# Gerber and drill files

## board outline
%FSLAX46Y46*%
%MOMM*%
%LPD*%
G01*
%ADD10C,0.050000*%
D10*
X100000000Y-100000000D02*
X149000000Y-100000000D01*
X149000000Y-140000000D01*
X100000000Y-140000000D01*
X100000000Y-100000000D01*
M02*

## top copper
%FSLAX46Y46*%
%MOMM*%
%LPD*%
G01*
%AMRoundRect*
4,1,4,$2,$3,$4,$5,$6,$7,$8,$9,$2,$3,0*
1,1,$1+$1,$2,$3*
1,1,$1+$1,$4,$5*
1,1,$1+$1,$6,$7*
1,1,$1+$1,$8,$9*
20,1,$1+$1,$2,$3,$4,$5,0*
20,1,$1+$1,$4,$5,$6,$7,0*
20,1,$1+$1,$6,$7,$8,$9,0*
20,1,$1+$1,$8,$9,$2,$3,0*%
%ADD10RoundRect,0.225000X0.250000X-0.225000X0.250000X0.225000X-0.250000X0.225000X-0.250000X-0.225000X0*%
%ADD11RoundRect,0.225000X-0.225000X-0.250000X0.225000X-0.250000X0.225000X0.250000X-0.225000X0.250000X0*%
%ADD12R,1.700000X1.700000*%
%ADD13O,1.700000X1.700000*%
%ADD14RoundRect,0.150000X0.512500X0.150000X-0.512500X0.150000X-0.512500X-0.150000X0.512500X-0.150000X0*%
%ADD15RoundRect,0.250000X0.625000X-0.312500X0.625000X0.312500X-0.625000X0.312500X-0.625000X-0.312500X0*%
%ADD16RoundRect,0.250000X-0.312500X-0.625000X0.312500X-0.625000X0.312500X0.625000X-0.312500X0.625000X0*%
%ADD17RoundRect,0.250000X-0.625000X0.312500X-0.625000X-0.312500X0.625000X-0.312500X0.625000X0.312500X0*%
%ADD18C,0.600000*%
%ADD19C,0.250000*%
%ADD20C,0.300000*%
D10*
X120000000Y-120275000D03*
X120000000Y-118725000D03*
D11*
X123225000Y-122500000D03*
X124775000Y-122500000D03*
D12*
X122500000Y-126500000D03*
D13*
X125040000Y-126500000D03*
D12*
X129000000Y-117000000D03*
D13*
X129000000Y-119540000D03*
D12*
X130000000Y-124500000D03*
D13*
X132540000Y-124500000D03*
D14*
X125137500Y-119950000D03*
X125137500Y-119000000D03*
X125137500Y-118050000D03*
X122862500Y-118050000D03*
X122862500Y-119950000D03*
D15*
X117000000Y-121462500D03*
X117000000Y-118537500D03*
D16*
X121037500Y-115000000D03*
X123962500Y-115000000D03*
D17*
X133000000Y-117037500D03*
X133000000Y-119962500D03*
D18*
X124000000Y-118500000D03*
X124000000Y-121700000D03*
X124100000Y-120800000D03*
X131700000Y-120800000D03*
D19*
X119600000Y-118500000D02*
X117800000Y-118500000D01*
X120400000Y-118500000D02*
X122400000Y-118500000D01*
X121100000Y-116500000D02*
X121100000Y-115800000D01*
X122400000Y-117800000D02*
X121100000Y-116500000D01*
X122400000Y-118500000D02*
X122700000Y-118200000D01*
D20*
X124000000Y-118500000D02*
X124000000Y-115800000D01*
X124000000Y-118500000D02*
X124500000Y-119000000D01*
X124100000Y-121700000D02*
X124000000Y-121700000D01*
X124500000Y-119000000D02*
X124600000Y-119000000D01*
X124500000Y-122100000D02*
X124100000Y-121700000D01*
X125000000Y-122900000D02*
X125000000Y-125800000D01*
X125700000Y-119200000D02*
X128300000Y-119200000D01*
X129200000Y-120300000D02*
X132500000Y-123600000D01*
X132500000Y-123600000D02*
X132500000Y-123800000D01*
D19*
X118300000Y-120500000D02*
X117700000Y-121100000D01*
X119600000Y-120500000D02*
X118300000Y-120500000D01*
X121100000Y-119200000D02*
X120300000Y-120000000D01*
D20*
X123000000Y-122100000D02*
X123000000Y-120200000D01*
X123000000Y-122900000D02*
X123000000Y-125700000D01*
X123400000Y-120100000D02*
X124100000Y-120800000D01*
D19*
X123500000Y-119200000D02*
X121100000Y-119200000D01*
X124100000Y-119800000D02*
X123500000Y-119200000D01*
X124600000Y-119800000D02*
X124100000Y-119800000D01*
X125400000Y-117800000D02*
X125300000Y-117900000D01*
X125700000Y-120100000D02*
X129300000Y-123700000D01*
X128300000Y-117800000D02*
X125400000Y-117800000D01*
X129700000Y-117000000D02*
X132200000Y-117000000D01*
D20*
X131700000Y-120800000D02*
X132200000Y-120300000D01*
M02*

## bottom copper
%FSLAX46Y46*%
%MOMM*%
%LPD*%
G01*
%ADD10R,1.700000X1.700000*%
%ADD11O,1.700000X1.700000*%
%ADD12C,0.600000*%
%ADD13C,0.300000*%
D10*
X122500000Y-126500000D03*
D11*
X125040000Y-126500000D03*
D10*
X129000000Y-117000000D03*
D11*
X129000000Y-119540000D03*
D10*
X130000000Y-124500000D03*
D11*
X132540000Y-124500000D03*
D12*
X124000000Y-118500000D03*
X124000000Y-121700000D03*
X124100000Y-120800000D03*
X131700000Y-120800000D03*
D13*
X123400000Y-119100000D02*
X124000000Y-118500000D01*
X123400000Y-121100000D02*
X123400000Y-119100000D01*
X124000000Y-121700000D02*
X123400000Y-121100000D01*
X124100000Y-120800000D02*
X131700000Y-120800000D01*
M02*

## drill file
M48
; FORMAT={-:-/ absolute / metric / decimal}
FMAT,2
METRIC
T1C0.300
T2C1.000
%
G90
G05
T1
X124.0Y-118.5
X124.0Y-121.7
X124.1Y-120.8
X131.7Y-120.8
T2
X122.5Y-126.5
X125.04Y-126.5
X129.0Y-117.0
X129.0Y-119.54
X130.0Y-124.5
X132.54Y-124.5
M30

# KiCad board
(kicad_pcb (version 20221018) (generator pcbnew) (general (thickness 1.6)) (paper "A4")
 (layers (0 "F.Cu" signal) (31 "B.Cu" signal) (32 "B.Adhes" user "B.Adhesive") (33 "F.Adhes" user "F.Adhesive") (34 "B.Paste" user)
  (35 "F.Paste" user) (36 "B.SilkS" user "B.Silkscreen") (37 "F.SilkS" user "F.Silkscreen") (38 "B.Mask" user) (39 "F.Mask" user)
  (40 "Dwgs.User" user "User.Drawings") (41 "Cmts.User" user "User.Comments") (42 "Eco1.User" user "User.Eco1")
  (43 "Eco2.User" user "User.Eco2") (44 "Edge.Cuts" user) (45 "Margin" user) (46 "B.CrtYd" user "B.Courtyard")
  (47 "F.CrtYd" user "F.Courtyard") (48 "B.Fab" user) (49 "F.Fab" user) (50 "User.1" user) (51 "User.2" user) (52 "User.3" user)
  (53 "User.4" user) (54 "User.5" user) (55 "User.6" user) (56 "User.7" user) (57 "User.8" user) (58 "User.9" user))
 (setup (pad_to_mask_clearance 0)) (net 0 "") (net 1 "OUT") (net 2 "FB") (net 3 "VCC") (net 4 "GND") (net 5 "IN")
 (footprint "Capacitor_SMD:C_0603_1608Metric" (layer "F.Cu") (at 120 119.5 90)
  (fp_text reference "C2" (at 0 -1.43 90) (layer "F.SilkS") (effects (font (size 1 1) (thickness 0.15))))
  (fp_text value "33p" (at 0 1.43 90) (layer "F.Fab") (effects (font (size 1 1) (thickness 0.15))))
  (pad "1" smd roundrect (at -0.775 0 90) (size 0.9 0.95) (layers "F.Cu" "F.Paste" "F.Mask") (roundrect_rratio 0.25) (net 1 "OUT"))
  (pad "2" smd roundrect (at 0.775 0 90) (size 0.9 0.95) (layers "F.Cu" "F.Paste" "F.Mask") (roundrect_rratio 0.25) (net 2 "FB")))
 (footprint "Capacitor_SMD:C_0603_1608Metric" (layer "F.Cu") (at 124 122.5)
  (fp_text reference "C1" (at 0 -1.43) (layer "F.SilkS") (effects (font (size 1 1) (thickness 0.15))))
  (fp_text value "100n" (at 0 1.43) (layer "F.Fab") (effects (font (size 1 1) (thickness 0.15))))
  (pad "1" smd roundrect (at -0.775 0) (size 0.9 0.95) (layers "F.Cu" "F.Paste" "F.Mask") (roundrect_rratio 0.25) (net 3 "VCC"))
  (pad "2" smd roundrect (at 0.775 0) (size 0.9 0.95) (layers "F.Cu" "F.Paste" "F.Mask") (roundrect_rratio 0.25) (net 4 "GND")))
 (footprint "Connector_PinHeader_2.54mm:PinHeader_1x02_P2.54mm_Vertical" (layer "F.Cu") (at 122.5 126.5 90)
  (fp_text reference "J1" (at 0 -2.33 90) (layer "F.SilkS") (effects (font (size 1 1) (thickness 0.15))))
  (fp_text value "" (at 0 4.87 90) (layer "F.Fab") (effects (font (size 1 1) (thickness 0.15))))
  (pad "1" thru_hole rect (at 0 0 90) (size 1.7 1.7) (drill 1) (layers "*.Cu" "*.Mask") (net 3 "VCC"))
  (pad "2" thru_hole oval (at 0 2.54 90) (size 1.7 1.7) (drill 1) (layers "*.Cu" "*.Mask") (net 4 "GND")))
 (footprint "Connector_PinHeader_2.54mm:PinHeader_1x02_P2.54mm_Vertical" (layer "F.Cu") (at 129 117)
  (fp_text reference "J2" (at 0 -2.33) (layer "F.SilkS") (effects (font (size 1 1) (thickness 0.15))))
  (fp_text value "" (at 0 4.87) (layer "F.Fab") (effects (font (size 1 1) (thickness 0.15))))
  (pad "1" thru_hole rect (at 0 0) (size 1.7 1.7) (drill 1) (layers "*.Cu" "*.Mask") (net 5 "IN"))
  (pad "2" thru_hole oval (at 0 2.54) (size 1.7 1.7) (drill 1) (layers "*.Cu" "*.Mask") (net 4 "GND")))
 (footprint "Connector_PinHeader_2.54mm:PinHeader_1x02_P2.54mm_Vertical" (layer "F.Cu") (at 130 124.5 90)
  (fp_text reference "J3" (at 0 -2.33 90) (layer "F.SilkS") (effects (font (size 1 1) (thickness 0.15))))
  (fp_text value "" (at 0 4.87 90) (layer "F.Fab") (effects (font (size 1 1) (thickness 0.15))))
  (pad "1" thru_hole rect (at 0 0 90) (size 1.7 1.7) (drill 1) (layers "*.Cu" "*.Mask") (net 1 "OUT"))
  (pad "2" thru_hole oval (at 0 2.54 90) (size 1.7 1.7) (drill 1) (layers "*.Cu" "*.Mask") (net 4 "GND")))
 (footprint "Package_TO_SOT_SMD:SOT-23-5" (layer "F.Cu") (at 124 119 180)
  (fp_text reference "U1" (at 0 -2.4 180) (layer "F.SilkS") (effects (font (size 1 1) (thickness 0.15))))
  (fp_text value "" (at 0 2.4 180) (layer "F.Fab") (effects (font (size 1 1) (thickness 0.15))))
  (pad "1" smd roundrect (at -1.1375 -0.95 180) (size 1.325 0.6) (layers "F.Cu" "F.Paste" "F.Mask") (roundrect_rratio 0.25) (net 1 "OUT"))
  (pad "2" smd roundrect (at -1.1375 0 180) (size 1.325 0.6) (layers "F.Cu" "F.Paste" "F.Mask") (roundrect_rratio 0.25) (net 4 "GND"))
  (pad "3" smd roundrect (at -1.1375 0.95 180) (size 1.325 0.6) (layers "F.Cu" "F.Paste" "F.Mask") (roundrect_rratio 0.25) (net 5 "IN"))
  (pad "4" smd roundrect (at 1.1375 0.95 180) (size 1.325 0.6) (layers "F.Cu" "F.Paste" "F.Mask") (roundrect_rratio 0.25) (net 2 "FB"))
  (pad "5" smd roundrect (at 1.1375 -0.95 180) (size 1.325 0.6) (layers "F.Cu" "F.Paste" "F.Mask") (roundrect_rratio 0.25) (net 3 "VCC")))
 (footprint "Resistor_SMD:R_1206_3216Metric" (layer "F.Cu") (at 117 120 90)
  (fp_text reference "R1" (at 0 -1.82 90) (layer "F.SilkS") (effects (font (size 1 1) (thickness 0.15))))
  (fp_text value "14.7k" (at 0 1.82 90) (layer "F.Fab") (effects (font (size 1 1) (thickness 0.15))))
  (pad "1" smd roundrect (at -1.4625 0 90) (size 1.125 1.75) (layers "F.Cu" "F.Paste" "F.Mask") (roundrect_rratio 0.222222) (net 1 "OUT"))
  (pad "2" smd roundrect (at 1.4625 0 90) (size 1.125 1.75) (layers "F.Cu" "F.Paste" "F.Mask") (roundrect_rratio 0.222222) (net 2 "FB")))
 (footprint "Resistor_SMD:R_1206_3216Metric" (layer "F.Cu") (at 122.5 115)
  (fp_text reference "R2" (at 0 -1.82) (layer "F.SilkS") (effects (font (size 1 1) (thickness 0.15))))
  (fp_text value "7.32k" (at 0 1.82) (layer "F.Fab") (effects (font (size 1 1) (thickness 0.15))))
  (pad "1" smd roundrect (at -1.4625 0) (size 1.125 1.75) (layers "F.Cu" "F.Paste" "F.Mask") (roundrect_rratio 0.222222) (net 2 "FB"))
  (pad "2" smd roundrect (at 1.4625 0) (size 1.125 1.75) (layers "F.Cu" "F.Paste" "F.Mask") (roundrect_rratio 0.222222) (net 4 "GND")))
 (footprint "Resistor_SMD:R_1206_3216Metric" (layer "F.Cu") (at 133 118.5 -90)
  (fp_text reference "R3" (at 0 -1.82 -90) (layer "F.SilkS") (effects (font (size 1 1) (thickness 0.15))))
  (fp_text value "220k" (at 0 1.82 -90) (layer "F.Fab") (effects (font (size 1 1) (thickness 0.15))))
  (pad "1" smd roundrect (at -1.4625 0 270) (size 1.125 1.75) (layers "F.Cu" "F.Paste" "F.Mask") (roundrect_rratio 0.222222) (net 5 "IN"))
  (pad "2" smd roundrect (at 1.4625 0 270) (size 1.125 1.75) (layers "F.Cu" "F.Paste" "F.Mask") (roundrect_rratio 0.222222) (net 3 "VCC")))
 (gr_rect (start 100 100) (end 149 140) (stroke (width 0.05) (type default)) (fill none) (layer "Edge.Cuts"))
 (segment (start 119.6 118.5) (end 117.8 118.5) (width 0.25) (layer "F.Cu") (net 2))
 (segment (start 120.4 118.5) (end 122.4 118.5) (width 0.25) (layer "F.Cu") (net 2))
 (segment (start 121.1 116.5) (end 121.1 115.8) (width 0.25) (layer "F.Cu") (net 2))
 (segment (start 122.4 117.8) (end 121.1 116.5) (width 0.25) (layer "F.Cu") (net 2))
 (segment (start 122.4 118.5) (end 122.7 118.2) (width 0.25) (layer "F.Cu") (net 2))
 (segment (start 124 118.5) (end 124 115.8) (width 0.3) (layer "F.Cu") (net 4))
 (segment (start 124 118.5) (end 124.5 119) (width 0.3) (layer "F.Cu") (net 4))
 (segment (start 124.1 121.7) (end 124 121.7) (width 0.3) (layer "F.Cu") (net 4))
 (segment (start 124.5 119) (end 124.6 119) (width 0.3) (layer "F.Cu") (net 4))
 (segment (start 124.5 122.1) (end 124.1 121.7) (width 0.3) (layer "F.Cu") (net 4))
 (segment (start 125 122.9) (end 125 125.8) (width 0.3) (layer "F.Cu") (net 4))
 (segment (start 125.7 119.2) (end 128.3 119.2) (width 0.3) (layer "F.Cu") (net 4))
 (segment (start 129.2 120.3) (end 132.5 123.6) (width 0.3) (layer "F.Cu") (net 4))
 (segment (start 132.5 123.6) (end 132.5 123.8) (width 0.3) (layer "F.Cu") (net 4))
 (via (at 124 118.5) (size 0.6) (drill 0.3) (layers "F.Cu" "B.Cu") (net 4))
 (via (at 124 121.7) (size 0.6) (drill 0.3) (layers "F.Cu" "B.Cu") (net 4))
 (segment (start 118.3 120.5) (end 117.7 121.1) (width 0.25) (layer "F.Cu") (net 1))
 (segment (start 119.6 120.5) (end 118.3 120.5) (width 0.25) (layer "F.Cu") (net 1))
 (segment (start 121.1 119.2) (end 120.3 120) (width 0.25) (layer "F.Cu") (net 1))
 (segment (start 123 122.1) (end 123 120.2) (width 0.3) (layer "F.Cu") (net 3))
 (segment (start 123 122.9) (end 123 125.7) (width 0.3) (layer "F.Cu") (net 3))
 (segment (start 123.4 119.1) (end 124 118.5) (width 0.3) (layer "B.Cu") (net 4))
 (segment (start 123.4 120.1) (end 124.1 120.8) (width 0.3) (layer "F.Cu") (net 3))
 (segment (start 123.4 121.1) (end 123.4 119.1) (width 0.3) (layer "B.Cu") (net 4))
 (segment (start 123.5 119.2) (end 121.1 119.2) (width 0.25) (layer "F.Cu") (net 1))
 (segment (start 124 121.7) (end 123.4 121.1) (width 0.3) (layer "B.Cu") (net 4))
 (segment (start 124.1 119.8) (end 123.5 119.2) (width 0.25) (layer "F.Cu") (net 1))
 (segment (start 124.6 119.8) (end 124.1 119.8) (width 0.25) (layer "F.Cu") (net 1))
 (segment (start 125.4 117.8) (end 125.3 117.9) (width 0.25) (layer "F.Cu") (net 5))
 (segment (start 125.7 120.1) (end 129.3 123.7) (width 0.25) (layer "F.Cu") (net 1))
 (segment (start 128.3 117.8) (end 125.4 117.8) (width 0.25) (layer "F.Cu") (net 5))
 (segment (start 129.7 117) (end 132.2 117) (width 0.25) (layer "F.Cu") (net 5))
 (segment (start 131.7 120.8) (end 132.2 120.3) (width 0.3) (layer "F.Cu") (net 3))
 (via (at 124.1 120.8) (size 0.6) (drill 0.3) (layers "F.Cu" "B.Cu") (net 3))
 (via (at 131.7 120.8) (size 0.6) (drill 0.3) (layers "F.Cu" "B.Cu") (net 3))
 (segment (start 124.1 120.8) (end 131.7 120.8) (width 0.3) (layer "B.Cu") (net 3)))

